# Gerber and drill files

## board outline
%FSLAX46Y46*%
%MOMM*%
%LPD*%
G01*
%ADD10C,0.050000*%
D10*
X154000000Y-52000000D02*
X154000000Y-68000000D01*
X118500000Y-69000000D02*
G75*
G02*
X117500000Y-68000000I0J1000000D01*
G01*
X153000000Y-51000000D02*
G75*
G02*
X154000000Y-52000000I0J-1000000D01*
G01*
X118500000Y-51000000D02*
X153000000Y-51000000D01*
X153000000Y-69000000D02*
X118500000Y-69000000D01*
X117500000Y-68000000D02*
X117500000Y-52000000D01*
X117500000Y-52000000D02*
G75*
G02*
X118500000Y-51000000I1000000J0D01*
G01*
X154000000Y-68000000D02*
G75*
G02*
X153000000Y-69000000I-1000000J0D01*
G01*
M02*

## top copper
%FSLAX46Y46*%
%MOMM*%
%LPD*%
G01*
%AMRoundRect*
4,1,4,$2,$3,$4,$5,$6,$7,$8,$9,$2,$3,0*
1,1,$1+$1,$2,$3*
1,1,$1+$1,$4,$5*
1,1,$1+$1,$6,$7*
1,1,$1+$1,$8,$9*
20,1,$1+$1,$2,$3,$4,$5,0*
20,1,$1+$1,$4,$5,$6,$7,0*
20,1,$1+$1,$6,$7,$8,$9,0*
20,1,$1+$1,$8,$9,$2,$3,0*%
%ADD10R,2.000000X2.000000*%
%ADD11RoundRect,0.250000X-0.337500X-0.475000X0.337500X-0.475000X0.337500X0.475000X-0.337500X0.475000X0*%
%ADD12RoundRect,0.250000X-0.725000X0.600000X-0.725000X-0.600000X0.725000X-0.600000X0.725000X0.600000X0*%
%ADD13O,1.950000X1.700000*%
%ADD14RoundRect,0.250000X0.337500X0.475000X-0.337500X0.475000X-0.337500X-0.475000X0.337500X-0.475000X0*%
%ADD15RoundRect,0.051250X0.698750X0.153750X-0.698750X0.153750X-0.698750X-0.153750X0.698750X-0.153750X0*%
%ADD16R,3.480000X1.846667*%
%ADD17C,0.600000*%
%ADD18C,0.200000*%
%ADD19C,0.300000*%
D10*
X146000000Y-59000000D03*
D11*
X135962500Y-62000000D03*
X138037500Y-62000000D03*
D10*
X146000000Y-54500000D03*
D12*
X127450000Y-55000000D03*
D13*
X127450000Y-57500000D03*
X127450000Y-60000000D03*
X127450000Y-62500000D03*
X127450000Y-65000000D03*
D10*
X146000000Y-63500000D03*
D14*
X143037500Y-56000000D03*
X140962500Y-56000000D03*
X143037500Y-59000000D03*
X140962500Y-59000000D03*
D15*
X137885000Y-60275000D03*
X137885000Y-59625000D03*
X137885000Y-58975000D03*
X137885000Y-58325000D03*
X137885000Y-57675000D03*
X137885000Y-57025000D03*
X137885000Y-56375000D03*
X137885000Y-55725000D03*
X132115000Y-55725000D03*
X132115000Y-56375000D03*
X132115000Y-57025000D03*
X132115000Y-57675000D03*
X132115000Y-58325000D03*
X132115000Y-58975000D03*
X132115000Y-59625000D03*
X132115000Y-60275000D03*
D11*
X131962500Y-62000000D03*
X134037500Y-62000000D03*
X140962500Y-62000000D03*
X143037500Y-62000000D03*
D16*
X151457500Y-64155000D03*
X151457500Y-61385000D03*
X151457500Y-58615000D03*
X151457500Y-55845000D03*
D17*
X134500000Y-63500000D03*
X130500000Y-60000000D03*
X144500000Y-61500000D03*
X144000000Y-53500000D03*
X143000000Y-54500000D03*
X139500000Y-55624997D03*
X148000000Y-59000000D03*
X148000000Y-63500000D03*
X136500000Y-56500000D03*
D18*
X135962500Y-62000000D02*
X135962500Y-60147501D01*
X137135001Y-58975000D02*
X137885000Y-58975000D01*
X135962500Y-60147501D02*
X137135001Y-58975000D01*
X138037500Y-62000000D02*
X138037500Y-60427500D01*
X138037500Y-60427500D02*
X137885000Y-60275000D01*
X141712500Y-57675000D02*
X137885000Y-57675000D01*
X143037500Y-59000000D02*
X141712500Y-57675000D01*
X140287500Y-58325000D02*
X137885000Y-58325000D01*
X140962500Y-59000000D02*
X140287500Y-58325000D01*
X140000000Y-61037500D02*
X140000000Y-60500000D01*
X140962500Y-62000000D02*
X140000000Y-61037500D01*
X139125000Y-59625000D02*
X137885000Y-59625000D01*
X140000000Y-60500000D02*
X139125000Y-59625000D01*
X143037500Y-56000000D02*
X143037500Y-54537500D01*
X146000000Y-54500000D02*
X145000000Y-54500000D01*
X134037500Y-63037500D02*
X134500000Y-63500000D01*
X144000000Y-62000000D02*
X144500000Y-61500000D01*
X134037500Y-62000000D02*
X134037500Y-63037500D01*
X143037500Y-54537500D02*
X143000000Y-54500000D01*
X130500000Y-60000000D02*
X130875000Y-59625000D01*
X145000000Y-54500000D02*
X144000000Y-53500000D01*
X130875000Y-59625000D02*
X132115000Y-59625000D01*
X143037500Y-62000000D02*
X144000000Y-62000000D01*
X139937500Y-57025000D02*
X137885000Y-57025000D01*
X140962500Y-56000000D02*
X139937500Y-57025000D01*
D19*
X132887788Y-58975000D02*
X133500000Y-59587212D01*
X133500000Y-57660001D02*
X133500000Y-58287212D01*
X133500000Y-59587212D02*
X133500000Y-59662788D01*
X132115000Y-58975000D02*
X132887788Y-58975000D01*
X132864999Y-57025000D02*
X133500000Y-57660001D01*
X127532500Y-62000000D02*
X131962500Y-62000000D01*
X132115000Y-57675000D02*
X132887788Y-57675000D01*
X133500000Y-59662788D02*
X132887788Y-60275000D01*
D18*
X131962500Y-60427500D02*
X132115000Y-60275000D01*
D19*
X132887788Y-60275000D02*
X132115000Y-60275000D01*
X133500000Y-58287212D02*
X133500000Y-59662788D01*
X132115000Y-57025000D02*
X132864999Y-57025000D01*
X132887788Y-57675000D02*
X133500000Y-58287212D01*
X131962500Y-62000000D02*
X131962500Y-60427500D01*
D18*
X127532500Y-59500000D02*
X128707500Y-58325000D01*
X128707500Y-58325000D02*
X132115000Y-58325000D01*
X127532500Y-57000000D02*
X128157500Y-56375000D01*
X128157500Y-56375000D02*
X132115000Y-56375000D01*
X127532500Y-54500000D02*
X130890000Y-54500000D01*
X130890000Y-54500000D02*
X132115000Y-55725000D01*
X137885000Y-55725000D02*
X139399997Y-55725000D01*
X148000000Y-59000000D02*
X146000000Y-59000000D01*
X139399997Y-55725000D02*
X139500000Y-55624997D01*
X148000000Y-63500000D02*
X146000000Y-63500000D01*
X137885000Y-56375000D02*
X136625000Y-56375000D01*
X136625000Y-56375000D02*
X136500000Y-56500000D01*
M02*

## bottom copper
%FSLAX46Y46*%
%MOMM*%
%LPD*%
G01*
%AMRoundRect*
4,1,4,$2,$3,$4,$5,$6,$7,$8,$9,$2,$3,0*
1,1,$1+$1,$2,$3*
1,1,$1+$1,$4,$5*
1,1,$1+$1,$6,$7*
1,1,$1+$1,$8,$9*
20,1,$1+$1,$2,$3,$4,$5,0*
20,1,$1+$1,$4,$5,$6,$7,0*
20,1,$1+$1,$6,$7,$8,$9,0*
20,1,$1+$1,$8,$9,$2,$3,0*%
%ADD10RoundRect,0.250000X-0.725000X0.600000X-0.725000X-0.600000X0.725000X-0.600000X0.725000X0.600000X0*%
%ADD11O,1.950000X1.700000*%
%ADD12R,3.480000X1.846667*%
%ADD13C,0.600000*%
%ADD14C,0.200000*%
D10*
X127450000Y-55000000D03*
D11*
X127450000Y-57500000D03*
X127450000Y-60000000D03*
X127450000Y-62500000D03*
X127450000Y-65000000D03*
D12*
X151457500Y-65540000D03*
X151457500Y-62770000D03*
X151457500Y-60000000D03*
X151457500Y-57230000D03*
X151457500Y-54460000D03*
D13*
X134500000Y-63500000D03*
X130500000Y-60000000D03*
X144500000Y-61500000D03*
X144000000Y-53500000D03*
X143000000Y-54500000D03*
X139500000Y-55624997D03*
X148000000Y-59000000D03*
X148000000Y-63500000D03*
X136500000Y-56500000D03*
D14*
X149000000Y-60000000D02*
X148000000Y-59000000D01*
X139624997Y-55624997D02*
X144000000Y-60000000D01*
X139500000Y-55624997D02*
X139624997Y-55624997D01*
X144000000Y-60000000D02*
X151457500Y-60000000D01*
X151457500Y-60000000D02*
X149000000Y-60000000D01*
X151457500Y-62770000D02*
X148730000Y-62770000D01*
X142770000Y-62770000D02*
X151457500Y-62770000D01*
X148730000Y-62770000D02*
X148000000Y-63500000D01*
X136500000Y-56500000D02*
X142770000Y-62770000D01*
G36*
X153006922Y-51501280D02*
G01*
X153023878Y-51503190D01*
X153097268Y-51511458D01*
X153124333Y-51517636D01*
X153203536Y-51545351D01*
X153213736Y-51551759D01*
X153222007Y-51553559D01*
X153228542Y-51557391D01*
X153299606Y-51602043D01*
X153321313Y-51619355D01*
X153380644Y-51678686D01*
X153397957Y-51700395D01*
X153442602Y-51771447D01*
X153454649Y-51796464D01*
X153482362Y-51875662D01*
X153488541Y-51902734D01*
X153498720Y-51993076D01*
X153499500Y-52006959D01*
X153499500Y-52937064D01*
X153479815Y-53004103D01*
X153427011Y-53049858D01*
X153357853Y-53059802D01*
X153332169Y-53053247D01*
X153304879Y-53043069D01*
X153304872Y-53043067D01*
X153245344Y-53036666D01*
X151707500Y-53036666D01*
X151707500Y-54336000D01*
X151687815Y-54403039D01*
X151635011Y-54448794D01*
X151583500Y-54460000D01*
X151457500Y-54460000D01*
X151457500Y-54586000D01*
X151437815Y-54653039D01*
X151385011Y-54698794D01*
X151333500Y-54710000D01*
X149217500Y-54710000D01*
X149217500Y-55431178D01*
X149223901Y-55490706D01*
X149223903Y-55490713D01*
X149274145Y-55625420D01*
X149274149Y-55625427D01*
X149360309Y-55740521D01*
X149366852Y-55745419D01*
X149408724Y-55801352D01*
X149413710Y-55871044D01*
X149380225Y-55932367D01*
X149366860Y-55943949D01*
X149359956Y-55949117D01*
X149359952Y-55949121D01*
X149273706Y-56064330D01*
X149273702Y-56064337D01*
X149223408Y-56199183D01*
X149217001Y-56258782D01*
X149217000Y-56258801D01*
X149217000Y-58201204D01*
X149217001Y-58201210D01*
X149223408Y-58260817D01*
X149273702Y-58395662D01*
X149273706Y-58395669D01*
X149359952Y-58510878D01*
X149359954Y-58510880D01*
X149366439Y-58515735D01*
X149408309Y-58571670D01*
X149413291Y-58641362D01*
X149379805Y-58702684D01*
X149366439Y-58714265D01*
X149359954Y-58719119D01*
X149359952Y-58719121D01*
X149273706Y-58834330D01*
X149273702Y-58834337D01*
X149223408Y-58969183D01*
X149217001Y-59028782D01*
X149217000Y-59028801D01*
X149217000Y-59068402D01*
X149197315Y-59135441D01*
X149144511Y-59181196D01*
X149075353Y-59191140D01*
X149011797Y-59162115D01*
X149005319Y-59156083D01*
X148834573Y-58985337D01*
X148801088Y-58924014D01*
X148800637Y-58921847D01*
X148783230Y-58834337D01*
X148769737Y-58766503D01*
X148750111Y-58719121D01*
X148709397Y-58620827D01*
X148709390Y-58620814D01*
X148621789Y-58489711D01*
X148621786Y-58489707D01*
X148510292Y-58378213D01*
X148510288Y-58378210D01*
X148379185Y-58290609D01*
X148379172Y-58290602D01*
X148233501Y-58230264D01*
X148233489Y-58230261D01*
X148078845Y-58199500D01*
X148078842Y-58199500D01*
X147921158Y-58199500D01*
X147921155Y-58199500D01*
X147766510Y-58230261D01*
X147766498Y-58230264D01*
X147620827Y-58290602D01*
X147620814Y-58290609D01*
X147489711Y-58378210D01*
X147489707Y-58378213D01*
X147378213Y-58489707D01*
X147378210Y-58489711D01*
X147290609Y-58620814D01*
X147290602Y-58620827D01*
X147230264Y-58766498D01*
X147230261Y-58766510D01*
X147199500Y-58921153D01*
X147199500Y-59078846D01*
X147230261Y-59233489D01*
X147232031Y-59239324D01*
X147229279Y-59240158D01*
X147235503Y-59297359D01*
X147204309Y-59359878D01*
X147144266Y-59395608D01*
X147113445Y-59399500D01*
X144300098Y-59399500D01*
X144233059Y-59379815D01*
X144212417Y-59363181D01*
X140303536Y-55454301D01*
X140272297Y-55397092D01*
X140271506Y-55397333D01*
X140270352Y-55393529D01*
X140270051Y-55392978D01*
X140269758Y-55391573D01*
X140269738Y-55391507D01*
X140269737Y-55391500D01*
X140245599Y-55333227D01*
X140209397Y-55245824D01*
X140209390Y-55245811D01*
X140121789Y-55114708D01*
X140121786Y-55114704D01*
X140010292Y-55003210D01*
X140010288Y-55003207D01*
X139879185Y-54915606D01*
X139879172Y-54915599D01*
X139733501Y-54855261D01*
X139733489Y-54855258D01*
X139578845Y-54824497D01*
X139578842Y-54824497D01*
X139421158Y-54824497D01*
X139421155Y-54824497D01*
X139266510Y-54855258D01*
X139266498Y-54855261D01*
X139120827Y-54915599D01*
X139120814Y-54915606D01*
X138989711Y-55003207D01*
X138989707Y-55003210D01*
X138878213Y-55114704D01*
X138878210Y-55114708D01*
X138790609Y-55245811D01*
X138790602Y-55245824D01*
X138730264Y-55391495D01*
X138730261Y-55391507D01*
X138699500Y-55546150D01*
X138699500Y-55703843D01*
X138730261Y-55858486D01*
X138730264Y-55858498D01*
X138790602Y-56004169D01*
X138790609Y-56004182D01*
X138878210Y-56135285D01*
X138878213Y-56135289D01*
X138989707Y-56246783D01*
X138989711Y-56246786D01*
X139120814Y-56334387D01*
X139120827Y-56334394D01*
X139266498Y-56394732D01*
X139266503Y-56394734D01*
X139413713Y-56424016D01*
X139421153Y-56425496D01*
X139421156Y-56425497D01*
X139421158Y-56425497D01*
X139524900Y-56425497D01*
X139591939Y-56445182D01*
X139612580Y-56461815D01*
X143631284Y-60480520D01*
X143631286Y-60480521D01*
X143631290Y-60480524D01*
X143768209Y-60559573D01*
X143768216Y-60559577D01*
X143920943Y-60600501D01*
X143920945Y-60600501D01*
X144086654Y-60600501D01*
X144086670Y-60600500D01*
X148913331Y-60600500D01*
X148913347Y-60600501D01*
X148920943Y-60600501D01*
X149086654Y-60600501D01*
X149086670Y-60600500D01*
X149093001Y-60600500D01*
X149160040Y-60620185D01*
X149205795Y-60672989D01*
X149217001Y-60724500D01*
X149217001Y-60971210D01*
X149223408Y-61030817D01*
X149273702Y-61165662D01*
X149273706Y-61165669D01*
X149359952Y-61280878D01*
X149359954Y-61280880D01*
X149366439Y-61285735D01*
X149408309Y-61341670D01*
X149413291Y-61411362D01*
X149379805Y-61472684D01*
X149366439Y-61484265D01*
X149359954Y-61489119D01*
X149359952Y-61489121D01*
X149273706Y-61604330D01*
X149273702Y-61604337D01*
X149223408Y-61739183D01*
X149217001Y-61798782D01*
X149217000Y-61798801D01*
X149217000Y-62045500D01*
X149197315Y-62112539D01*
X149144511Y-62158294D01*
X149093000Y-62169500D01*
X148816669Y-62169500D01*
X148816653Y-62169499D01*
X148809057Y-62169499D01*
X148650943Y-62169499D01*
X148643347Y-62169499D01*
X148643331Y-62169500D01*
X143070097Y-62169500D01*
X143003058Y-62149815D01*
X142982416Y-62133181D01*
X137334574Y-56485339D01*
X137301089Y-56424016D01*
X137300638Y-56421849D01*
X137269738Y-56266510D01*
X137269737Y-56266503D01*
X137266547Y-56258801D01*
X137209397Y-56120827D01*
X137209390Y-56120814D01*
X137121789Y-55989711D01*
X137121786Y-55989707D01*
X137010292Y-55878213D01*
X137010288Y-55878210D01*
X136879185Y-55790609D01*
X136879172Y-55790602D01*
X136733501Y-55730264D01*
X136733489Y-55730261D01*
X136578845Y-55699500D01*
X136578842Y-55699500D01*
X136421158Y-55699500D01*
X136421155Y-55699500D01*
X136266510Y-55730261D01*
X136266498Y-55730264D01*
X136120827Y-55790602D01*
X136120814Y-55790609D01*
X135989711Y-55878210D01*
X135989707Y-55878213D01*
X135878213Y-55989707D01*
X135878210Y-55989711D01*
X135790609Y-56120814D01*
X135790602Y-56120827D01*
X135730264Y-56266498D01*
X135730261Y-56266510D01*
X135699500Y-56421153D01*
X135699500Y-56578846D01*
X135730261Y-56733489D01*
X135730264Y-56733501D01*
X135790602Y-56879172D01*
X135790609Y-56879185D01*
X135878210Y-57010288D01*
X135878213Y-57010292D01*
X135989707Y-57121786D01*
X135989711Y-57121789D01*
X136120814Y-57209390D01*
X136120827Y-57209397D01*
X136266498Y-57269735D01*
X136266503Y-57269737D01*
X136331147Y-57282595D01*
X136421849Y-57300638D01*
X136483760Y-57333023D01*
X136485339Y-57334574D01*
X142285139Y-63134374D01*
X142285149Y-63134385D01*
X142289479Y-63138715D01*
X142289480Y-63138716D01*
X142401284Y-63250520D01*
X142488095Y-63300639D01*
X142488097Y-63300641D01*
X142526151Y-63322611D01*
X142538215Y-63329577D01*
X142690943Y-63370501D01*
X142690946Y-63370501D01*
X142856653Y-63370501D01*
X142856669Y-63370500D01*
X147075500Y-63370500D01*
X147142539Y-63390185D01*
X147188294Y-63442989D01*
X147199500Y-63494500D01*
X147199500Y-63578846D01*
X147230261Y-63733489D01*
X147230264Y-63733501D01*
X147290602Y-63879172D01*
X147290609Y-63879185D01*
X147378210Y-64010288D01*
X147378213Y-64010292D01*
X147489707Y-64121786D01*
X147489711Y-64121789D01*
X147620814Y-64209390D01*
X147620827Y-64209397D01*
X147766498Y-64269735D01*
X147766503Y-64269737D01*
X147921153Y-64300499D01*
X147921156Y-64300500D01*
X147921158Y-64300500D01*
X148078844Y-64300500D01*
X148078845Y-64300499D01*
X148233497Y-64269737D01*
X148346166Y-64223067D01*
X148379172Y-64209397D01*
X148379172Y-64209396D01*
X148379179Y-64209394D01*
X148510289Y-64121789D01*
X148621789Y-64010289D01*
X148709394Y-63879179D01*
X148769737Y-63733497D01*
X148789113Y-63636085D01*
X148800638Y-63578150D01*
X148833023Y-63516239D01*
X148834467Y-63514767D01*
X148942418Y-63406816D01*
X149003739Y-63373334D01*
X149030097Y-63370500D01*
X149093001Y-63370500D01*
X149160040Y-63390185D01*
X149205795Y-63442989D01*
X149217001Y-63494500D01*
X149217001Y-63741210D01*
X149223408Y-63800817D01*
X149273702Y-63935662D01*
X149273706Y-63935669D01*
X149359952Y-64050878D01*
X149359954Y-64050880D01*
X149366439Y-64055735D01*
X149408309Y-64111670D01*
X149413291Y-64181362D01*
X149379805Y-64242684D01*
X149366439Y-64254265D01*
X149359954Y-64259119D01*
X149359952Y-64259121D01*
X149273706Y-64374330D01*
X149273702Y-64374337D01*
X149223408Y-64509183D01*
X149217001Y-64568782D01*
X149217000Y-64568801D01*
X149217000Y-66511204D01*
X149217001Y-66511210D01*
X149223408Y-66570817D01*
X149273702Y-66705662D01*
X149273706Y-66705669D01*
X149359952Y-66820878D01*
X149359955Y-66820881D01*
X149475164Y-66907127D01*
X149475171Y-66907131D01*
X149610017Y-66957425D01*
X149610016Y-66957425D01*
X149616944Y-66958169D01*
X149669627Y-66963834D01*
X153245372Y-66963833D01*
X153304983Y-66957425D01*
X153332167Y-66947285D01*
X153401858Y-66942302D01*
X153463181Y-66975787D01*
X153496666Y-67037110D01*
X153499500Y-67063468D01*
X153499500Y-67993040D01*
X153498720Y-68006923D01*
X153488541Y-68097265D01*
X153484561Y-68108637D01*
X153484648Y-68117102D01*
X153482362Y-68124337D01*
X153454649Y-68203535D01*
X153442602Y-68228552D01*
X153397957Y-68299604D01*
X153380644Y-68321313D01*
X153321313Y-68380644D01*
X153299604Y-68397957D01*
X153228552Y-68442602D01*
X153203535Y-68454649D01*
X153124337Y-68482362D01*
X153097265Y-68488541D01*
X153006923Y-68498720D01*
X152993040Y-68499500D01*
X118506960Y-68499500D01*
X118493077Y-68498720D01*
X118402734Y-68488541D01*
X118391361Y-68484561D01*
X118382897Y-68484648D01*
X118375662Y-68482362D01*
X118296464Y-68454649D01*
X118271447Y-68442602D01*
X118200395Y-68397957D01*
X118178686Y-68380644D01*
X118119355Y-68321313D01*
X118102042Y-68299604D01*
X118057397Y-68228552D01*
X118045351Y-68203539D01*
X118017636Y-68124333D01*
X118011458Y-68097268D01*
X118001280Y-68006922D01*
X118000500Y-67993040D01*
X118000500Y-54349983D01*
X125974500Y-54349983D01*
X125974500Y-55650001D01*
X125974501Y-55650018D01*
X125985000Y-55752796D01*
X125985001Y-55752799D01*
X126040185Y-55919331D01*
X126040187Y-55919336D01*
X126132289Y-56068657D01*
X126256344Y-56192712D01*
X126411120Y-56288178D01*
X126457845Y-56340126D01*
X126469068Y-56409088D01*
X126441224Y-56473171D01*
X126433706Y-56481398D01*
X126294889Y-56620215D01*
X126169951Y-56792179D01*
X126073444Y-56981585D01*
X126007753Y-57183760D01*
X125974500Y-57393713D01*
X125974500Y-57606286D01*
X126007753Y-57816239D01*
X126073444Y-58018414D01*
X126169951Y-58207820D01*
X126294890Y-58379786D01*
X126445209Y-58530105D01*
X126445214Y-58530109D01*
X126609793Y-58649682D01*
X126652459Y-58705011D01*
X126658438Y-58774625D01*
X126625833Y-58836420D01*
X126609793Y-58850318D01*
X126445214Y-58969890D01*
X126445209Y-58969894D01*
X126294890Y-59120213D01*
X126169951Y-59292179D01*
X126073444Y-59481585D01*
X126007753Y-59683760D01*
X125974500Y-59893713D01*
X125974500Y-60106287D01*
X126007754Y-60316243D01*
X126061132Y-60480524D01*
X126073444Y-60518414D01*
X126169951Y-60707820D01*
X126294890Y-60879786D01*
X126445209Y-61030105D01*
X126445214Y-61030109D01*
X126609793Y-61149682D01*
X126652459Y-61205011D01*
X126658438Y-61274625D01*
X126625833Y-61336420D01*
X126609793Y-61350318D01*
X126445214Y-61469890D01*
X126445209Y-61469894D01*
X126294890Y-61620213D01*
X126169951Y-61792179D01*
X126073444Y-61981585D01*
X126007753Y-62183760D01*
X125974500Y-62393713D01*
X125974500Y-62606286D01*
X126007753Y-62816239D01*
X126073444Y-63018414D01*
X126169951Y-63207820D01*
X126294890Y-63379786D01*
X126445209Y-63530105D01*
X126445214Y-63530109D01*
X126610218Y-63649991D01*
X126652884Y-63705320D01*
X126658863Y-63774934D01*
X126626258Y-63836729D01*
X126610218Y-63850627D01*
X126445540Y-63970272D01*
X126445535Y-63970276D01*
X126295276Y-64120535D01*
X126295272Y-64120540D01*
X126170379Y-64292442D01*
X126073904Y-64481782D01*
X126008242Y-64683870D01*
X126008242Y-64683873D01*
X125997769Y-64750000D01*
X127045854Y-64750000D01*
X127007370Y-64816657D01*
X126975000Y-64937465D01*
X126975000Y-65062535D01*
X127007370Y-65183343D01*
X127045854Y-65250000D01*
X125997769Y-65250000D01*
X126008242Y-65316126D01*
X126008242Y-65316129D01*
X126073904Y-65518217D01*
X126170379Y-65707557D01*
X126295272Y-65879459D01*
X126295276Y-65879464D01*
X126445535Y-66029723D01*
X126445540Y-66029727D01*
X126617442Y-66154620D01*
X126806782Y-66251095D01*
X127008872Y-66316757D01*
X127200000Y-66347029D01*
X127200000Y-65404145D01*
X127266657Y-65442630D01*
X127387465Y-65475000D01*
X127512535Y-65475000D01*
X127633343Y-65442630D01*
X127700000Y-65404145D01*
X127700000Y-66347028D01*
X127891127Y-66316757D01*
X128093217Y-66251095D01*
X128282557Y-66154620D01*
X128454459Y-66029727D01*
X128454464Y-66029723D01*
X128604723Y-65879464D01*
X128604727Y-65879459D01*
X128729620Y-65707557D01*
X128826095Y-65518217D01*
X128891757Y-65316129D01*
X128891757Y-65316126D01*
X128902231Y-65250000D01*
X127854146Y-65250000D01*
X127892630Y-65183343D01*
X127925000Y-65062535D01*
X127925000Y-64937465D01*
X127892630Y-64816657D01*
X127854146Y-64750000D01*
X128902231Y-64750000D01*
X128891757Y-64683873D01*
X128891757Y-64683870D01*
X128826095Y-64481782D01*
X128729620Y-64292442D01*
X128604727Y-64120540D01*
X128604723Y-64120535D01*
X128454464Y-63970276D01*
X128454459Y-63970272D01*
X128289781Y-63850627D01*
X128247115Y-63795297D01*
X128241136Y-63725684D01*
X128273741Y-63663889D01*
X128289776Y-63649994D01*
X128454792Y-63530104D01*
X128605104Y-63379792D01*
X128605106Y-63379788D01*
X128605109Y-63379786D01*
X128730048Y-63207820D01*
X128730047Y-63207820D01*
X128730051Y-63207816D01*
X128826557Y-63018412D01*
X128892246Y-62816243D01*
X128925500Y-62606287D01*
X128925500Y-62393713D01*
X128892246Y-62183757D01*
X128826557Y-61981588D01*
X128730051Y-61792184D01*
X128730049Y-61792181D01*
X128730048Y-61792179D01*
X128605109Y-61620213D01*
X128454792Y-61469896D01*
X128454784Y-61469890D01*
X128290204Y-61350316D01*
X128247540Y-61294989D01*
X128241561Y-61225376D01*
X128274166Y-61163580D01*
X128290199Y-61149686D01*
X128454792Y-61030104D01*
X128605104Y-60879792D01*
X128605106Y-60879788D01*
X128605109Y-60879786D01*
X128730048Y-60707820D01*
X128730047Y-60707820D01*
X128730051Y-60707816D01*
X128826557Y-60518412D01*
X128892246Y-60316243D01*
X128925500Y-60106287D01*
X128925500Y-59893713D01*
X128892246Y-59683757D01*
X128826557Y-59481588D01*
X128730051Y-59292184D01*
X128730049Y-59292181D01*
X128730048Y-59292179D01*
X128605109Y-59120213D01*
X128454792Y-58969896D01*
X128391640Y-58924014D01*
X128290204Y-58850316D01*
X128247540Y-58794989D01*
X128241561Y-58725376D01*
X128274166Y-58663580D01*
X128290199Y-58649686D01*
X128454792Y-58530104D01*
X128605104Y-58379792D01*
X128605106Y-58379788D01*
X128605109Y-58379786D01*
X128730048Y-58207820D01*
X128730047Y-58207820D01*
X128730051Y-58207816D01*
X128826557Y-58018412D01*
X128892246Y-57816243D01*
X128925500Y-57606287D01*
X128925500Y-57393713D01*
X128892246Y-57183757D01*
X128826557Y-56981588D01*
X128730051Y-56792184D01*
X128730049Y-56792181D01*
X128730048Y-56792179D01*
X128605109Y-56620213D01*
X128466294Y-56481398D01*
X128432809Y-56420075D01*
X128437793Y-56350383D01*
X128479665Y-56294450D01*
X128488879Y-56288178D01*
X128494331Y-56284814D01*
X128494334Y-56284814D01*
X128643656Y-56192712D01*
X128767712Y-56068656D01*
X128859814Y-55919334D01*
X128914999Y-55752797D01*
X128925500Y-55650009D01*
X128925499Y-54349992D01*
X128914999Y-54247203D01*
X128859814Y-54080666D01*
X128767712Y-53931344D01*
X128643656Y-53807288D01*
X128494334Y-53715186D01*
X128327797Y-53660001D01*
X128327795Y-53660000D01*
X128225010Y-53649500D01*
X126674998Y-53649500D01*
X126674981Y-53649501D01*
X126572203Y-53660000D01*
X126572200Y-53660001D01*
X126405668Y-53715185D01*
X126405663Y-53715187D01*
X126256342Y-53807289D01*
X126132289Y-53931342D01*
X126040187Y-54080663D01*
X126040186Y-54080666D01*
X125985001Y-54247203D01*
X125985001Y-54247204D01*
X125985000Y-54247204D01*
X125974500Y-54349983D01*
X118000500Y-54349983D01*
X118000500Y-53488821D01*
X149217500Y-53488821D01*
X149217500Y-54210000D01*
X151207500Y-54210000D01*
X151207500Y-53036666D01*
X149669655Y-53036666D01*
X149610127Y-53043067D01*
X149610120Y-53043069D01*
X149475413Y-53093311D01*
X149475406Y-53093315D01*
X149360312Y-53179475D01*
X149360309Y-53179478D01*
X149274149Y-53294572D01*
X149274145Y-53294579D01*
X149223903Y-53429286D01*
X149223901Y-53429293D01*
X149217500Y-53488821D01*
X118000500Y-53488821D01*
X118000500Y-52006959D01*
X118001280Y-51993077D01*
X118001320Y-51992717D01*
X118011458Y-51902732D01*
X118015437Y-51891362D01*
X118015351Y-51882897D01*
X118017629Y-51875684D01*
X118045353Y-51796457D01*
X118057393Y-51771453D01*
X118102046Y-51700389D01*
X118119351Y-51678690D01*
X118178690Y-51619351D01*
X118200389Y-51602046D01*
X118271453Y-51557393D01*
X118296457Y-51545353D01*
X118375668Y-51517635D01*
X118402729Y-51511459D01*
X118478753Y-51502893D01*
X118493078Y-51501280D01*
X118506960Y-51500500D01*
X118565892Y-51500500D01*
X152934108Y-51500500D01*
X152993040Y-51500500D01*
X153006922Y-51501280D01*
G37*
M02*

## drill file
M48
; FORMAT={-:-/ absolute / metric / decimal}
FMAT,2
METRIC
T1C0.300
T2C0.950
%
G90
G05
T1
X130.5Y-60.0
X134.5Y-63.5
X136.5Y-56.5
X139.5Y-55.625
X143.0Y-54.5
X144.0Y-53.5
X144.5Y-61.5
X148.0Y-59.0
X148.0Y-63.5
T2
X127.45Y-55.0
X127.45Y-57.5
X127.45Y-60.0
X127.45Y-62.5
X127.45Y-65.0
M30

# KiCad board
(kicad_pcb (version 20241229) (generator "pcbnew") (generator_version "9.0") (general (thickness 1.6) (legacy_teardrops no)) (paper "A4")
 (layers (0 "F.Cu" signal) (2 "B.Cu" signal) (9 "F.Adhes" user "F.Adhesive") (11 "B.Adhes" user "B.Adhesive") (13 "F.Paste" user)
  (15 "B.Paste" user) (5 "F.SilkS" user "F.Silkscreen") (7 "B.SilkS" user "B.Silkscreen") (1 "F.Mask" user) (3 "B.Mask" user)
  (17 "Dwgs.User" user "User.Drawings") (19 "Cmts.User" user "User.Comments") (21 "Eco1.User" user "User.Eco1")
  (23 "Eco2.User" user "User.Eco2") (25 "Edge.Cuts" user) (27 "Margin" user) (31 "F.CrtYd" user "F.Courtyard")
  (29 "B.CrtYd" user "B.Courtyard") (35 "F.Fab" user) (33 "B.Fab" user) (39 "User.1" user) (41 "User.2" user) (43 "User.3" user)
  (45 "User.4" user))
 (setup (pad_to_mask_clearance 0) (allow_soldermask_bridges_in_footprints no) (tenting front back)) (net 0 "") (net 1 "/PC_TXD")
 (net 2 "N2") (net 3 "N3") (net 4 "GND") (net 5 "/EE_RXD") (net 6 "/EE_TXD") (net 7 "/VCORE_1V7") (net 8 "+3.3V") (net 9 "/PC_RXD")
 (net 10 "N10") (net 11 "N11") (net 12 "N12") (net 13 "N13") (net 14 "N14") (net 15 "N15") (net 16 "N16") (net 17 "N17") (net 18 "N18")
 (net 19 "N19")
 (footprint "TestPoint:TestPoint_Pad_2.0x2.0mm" (layer "F.Cu") (at 146 59)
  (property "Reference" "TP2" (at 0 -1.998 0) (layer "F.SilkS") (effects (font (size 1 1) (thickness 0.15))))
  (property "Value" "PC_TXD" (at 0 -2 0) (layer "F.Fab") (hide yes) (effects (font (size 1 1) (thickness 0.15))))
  (pad "1" smd rect (at 0 0) (size 2 2) (layers "F.Cu" "F.Mask") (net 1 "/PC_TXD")))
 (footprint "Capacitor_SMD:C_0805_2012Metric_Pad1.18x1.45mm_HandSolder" (layer "F.Cu") (at 137 62)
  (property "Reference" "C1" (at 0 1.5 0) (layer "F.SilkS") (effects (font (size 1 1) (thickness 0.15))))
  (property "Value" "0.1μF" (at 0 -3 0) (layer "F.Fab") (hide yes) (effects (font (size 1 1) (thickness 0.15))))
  (pad "1" smd roundrect (at -1.0375 0) (size 1.175 1.45) (layers "F.Cu" "F.Mask" "F.Paste") (roundrect_rratio 0.212766) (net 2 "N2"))
  (pad "2" smd roundrect (at 1.0375 0) (size 1.175 1.45) (layers "F.Cu" "F.Mask" "F.Paste") (roundrect_rratio 0.212766) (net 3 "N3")))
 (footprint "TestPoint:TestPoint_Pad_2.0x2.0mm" (layer "F.Cu") (at 146 54.5)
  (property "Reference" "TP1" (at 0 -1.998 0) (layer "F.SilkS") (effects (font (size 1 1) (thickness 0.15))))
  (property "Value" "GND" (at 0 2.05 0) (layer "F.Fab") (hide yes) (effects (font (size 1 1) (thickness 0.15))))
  (pad "1" smd rect (at 0 0) (size 2 2) (layers "F.Cu" "F.Mask") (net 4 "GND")))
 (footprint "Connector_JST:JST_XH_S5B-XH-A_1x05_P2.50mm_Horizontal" (layer "F.Cu") (at 127.45 55 -90)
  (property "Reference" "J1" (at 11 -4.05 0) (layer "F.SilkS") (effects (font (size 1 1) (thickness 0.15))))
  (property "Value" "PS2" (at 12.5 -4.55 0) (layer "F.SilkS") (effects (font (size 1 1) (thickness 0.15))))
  (pad "1" thru_hole roundrect (at 0 0 270) (size 1.7 1.95) (drill 0.95) (layers "*.Cu" "*.Mask") (remove_unused_layers no)
   (roundrect_rratio 0.147059) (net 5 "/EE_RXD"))
  (pad "2" thru_hole oval (at 2.5 0 270) (size 1.7 1.95) (drill 0.95) (layers "*.Cu" "*.Mask") (remove_unused_layers no) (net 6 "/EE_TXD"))
  (pad "3" thru_hole oval (at 5 0 270) (size 1.7 1.95) (drill 0.95) (layers "*.Cu" "*.Mask") (remove_unused_layers no) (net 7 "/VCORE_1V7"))
  (pad "4" thru_hole oval (at 7.5 0 270) (size 1.7 1.95) (drill 0.95) (layers "*.Cu" "*.Mask") (remove_unused_layers no) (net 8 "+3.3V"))
  (pad "5" thru_hole oval (at 10 0 270) (size 1.7 1.95) (drill 0.95) (layers "*.Cu" "*.Mask") (remove_unused_layers no) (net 4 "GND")))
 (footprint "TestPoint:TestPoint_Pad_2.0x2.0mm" (layer "F.Cu") (at 146 63.5)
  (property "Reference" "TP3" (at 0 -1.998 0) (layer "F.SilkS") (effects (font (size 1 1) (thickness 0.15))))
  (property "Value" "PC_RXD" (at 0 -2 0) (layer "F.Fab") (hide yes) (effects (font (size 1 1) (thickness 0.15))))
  (pad "1" smd rect (at 0 0) (size 2 2) (layers "F.Cu" "F.Mask") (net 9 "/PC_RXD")))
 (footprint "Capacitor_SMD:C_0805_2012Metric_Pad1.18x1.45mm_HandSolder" (layer "F.Cu") (at 142 56 180)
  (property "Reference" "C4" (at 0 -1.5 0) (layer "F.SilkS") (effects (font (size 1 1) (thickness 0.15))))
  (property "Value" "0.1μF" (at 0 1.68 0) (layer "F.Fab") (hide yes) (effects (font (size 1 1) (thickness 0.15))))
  (pad "1" smd roundrect (at -1.0375 0 180) (size 1.175 1.45) (layers "F.Cu" "F.Mask" "F.Paste") (roundrect_rratio 0.212766) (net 4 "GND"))
  (pad "2" smd roundrect (at 1.0375 0 180) (size 1.175 1.45) (layers "F.Cu" "F.Mask" "F.Paste") (roundrect_rratio 0.212766) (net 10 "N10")))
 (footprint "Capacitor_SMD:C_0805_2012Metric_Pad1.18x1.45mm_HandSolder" (layer "F.Cu") (at 142 59 180)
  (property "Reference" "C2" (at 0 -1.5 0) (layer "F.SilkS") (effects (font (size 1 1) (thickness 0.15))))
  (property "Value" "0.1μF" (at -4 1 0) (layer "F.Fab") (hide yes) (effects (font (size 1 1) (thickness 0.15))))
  (pad "1" smd roundrect (at -1.0375 0 180) (size 1.175 1.45) (layers "F.Cu" "F.Mask" "F.Paste") (roundrect_rratio 0.212766) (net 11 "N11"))
  (pad "2" smd roundrect (at 1.0375 0 180) (size 1.175 1.45) (layers "F.Cu" "F.Mask" "F.Paste") (roundrect_rratio 0.212766) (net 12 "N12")))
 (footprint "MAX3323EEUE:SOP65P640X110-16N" (layer "F.Cu") (at 135 58 180)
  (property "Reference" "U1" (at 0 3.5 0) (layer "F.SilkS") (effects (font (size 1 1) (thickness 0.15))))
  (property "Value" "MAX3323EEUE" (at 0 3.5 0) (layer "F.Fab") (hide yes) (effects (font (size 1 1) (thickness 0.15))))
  (pad "1" smd roundrect (at -2.885 -2.275 180) (size 1.5 0.41) (layers "F.Cu" "F.Mask" "F.Paste") (roundrect_rratio 0.125) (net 3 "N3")
   (solder_mask_margin 0.102))
  (pad "2" smd roundrect (at -2.885 -1.625 180) (size 1.5 0.41) (layers "F.Cu" "F.Mask" "F.Paste") (roundrect_rratio 0.125) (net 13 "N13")
   (solder_mask_margin 0.102))
  (pad "3" smd roundrect (at -2.885 -0.975 180) (size 1.5 0.41) (layers "F.Cu" "F.Mask" "F.Paste") (roundrect_rratio 0.125) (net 2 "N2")
   (solder_mask_margin 0.102))
  (pad "4" smd roundrect (at -2.885 -0.325 180) (size 1.5 0.41) (layers "F.Cu" "F.Mask" "F.Paste") (roundrect_rratio 0.125) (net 12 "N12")
   (solder_mask_margin 0.102))
  (pad "5" smd roundrect (at -2.885 0.325 180) (size 1.5 0.41) (layers "F.Cu" "F.Mask" "F.Paste") (roundrect_rratio 0.125) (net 11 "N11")
   (solder_mask_margin 0.102))
  (pad "6" smd roundrect (at -2.885 0.975 180) (size 1.5 0.41) (layers "F.Cu" "F.Mask" "F.Paste") (roundrect_rratio 0.125) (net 10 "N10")
   (solder_mask_margin 0.102))
  (pad "7" smd roundrect (at -2.885 1.625 180) (size 1.5 0.41) (layers "F.Cu" "F.Mask" "F.Paste") (roundrect_rratio 0.125) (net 9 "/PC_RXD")
   (solder_mask_margin 0.102))
  (pad "8" smd roundrect (at -2.885 2.275 180) (size 1.5 0.41) (layers "F.Cu" "F.Mask" "F.Paste") (roundrect_rratio 0.125) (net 1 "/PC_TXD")
   (solder_mask_margin 0.102))
  (pad "9" smd roundrect (at 2.885 2.275 180) (size 1.5 0.41) (layers "F.Cu" "F.Mask" "F.Paste") (roundrect_rratio 0.125) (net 5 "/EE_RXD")
   (solder_mask_margin 0.102))
  (pad "10" smd roundrect (at 2.885 1.625 180) (size 1.5 0.41) (layers "F.Cu" "F.Mask" "F.Paste") (roundrect_rratio 0.125) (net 6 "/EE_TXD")
   (solder_mask_margin 0.102))
  (pad "11" smd roundrect (at 2.885 0.975 180) (size 1.5 0.41) (layers "F.Cu" "F.Mask" "F.Paste") (roundrect_rratio 0.125) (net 8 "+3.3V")
   (solder_mask_margin 0.102))
  (pad "12" smd roundrect (at 2.885 0.325 180) (size 1.5 0.41) (layers "F.Cu" "F.Mask" "F.Paste") (roundrect_rratio 0.125) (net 8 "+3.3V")
   (solder_mask_margin 0.102))
  (pad "13" smd roundrect (at 2.885 -0.325 180) (size 1.5 0.41) (layers "F.Cu" "F.Mask" "F.Paste") (roundrect_rratio 0.125)
   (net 7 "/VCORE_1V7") (solder_mask_margin 0.102))
  (pad "14" smd roundrect (at 2.885 -0.975 180) (size 1.5 0.41) (layers "F.Cu" "F.Mask" "F.Paste") (roundrect_rratio 0.125) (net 8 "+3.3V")
   (solder_mask_margin 0.102))
  (pad "15" smd roundrect (at 2.885 -1.625 180) (size 1.5 0.41) (layers "F.Cu" "F.Mask" "F.Paste") (roundrect_rratio 0.125) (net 4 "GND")
   (solder_mask_margin 0.102))
  (pad "16" smd roundrect (at 2.885 -2.275 180) (size 1.5 0.41) (layers "F.Cu" "F.Mask" "F.Paste") (roundrect_rratio 0.125) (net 8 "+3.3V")
   (solder_mask_margin 0.102)))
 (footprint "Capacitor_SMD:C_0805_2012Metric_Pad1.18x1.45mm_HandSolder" (layer "F.Cu") (at 133 62)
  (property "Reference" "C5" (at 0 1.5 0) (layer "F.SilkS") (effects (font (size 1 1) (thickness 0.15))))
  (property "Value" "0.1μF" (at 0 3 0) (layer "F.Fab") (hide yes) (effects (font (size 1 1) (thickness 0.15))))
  (pad "1" smd roundrect (at -1.0375 0) (size 1.175 1.45) (layers "F.Cu" "F.Mask" "F.Paste") (roundrect_rratio 0.212766) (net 8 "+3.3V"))
  (pad "2" smd roundrect (at 1.0375 0) (size 1.175 1.45) (layers "F.Cu" "F.Mask" "F.Paste") (roundrect_rratio 0.212766) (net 4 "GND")))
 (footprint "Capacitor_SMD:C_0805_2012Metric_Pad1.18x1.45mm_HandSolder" (layer "F.Cu") (at 142 62)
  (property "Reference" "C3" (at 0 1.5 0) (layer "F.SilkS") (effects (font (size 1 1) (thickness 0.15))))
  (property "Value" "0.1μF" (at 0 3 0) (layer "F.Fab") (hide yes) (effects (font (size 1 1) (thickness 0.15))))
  (pad "1" smd roundrect (at -1.0375 0) (size 1.175 1.45) (layers "F.Cu" "F.Mask" "F.Paste") (roundrect_rratio 0.212766) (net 13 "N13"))
  (pad "2" smd roundrect (at 1.0375 0) (size 1.175 1.45) (layers "F.Cu" "F.Mask" "F.Paste") (roundrect_rratio 0.212766) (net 4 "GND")))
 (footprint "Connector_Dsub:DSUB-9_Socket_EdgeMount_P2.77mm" (layer "B.Cu") (at 151.4575 60 -90)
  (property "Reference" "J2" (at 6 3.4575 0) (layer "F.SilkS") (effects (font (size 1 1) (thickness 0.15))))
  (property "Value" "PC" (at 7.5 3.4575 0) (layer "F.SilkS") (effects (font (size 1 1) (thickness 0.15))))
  (pad "1" smd rect (at 5.54 0 270) (size 1.846667 3.48) (layers "B.Cu" "B.Mask" "B.Paste") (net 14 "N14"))
  (pad "2" smd rect (at 2.77 0 270) (size 1.846667 3.48) (layers "B.Cu" "B.Mask" "B.Paste") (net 9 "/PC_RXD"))
  (pad "3" smd rect (at 0 0 270) (size 1.846667 3.48) (layers "B.Cu" "B.Mask" "B.Paste") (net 1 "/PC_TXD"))
  (pad "4" smd rect (at -2.77 0 270) (size 1.846667 3.48) (layers "B.Cu" "B.Mask" "B.Paste") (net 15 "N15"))
  (pad "5" smd rect (at -5.54 0 270) (size 1.846667 3.48) (layers "B.Cu" "B.Mask" "B.Paste") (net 4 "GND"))
  (pad "6" smd rect (at 4.155 0 270) (size 1.846667 3.48) (layers "F.Cu" "F.Mask" "F.Paste") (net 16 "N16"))
  (pad "7" smd rect (at 1.385 0 270) (size 1.846667 3.48) (layers "F.Cu" "F.Mask" "F.Paste") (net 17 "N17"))
  (pad "8" smd rect (at -1.385 0 270) (size 1.846667 3.48) (layers "F.Cu" "F.Mask" "F.Paste") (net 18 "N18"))
  (pad "9" smd rect (at -4.155 0 270) (size 1.846667 3.48) (layers "F.Cu" "F.Mask" "F.Paste") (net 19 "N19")))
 (gr_line (start 154 52) (end 154 68) (stroke (width 0.05) (type default)) (layer "Edge.Cuts"))
 (gr_arc (start 118.5 69) (mid 117.792893 68.707107) (end 117.5 68) (stroke (width 0.05) (type default)) (layer "Edge.Cuts"))
 (gr_arc (start 153 51) (mid 153.707107 51.292893) (end 154 52) (stroke (width 0.05) (type default)) (layer "Edge.Cuts"))
 (gr_line (start 118.5 51) (end 153 51) (stroke (width 0.05) (type default)) (layer "Edge.Cuts"))
 (gr_line (start 153 69) (end 118.5 69) (stroke (width 0.05) (type default)) (layer "Edge.Cuts"))
 (gr_line (start 117.5 68) (end 117.5 52) (stroke (width 0.05) (type default)) (layer "Edge.Cuts"))
 (gr_arc (start 117.5 52) (mid 117.792893 51.292893) (end 118.5 51) (stroke (width 0.05) (type default)) (layer "Edge.Cuts"))
 (gr_arc (start 154 68) (mid 153.707107 68.707107) (end 153 69) (stroke (width 0.05) (type default)) (layer "Edge.Cuts"))
 (segment (start 135.9625 62) (end 135.9625 60.147501) (width 0.2) (layer "F.Cu") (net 2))
 (segment (start 137.135001 58.975) (end 137.885 58.975) (width 0.2) (layer "F.Cu") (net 2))
 (segment (start 135.9625 60.147501) (end 137.135001 58.975) (width 0.2) (layer "F.Cu") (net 2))
 (segment (start 138.0375 62) (end 138.0375 60.4275) (width 0.2) (layer "F.Cu") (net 3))
 (segment (start 138.0375 60.4275) (end 137.885 60.275) (width 0.2) (layer "F.Cu") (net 3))
 (segment (start 141.7125 57.675) (end 137.885 57.675) (width 0.2) (layer "F.Cu") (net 11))
 (segment (start 143.0375 59) (end 141.7125 57.675) (width 0.2) (layer "F.Cu") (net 11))
 (segment (start 140.2875 58.325) (end 137.885 58.325) (width 0.2) (layer "F.Cu") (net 12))
 (segment (start 140.9625 59) (end 140.2875 58.325) (width 0.2) (layer "F.Cu") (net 12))
 (segment (start 140 61.0375) (end 140 60.5) (width 0.2) (layer "F.Cu") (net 13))
 (segment (start 140.9625 62) (end 140 61.0375) (width 0.2) (layer "F.Cu") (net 13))
 (segment (start 139.125 59.625) (end 137.885 59.625) (width 0.2) (layer "F.Cu") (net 13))
 (segment (start 140 60.5) (end 139.125 59.625) (width 0.2) (layer "F.Cu") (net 13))
 (segment (start 143.0375 56) (end 143.0375 54.5375) (width 0.2) (layer "F.Cu") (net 4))
 (segment (start 146 54.5) (end 145 54.5) (width 0.2) (layer "F.Cu") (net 4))
 (segment (start 134.0375 63.0375) (end 134.5 63.5) (width 0.2) (layer "F.Cu") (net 4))
 (segment (start 144 62) (end 144.5 61.5) (width 0.2) (layer "F.Cu") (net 4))
 (segment (start 134.0375 62) (end 134.0375 63.0375) (width 0.2) (layer "F.Cu") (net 4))
 (segment (start 143.0375 54.5375) (end 143 54.5) (width 0.2) (layer "F.Cu") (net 4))
 (segment (start 130.5 60) (end 130.875 59.625) (width 0.2) (layer "F.Cu") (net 4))
 (segment (start 145 54.5) (end 144 53.5) (width 0.2) (layer "F.Cu") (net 4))
 (segment (start 130.875 59.625) (end 132.115 59.625) (width 0.2) (layer "F.Cu") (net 4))
 (segment (start 143.0375 62) (end 144 62) (width 0.2) (layer "F.Cu") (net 4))
 (via (at 134.5 63.5) (size 0.6) (drill 0.3) (layers "F.Cu" "B.Cu") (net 4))
 (via (at 130.5 60) (size 0.6) (drill 0.3) (layers "F.Cu" "B.Cu") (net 4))
 (via (at 144.5 61.5) (size 0.6) (drill 0.3) (layers "F.Cu" "B.Cu") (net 4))
 (via (at 144 53.5) (size 0.6) (drill 0.3) (layers "F.Cu" "B.Cu") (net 4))
 (via (at 143 54.5) (size 0.6) (drill 0.3) (layers "F.Cu" "B.Cu") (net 4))
 (segment (start 139.9375 57.025) (end 137.885 57.025) (width 0.2) (layer "F.Cu") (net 10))
 (segment (start 140.9625 56) (end 139.9375 57.025) (width 0.2) (layer "F.Cu") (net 10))
 (segment (start 132.887788 58.975) (end 133.5 59.587212) (width 0.3) (layer "F.Cu") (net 8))
 (segment (start 133.5 57.660001) (end 133.5 58.287212) (width 0.3) (layer "F.Cu") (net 8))
 (segment (start 133.5 59.587212) (end 133.5 59.662788) (width 0.3) (layer "F.Cu") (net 8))
 (segment (start 132.115 58.975) (end 132.887788 58.975) (width 0.3) (layer "F.Cu") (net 8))
 (segment (start 132.864999 57.025) (end 133.5 57.660001) (width 0.3) (layer "F.Cu") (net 8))
 (segment (start 127.5325 62) (end 131.9625 62) (width 0.3) (layer "F.Cu") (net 8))
 (segment (start 132.115 57.675) (end 132.887788 57.675) (width 0.3) (layer "F.Cu") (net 8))
 (segment (start 133.5 59.662788) (end 132.887788 60.275) (width 0.3) (layer "F.Cu") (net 8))
 (segment (start 131.9625 60.4275) (end 132.115 60.275) (width 0.2) (layer "F.Cu") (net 8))
 (segment (start 132.887788 60.275) (end 132.115 60.275) (width 0.3) (layer "F.Cu") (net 8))
 (segment (start 133.5 58.287212) (end 133.5 59.662788) (width 0.3) (layer "F.Cu") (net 8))
 (segment (start 132.115 57.025) (end 132.864999 57.025) (width 0.3) (layer "F.Cu") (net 8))
 (segment (start 132.887788 57.675) (end 133.5 58.287212) (width 0.3) (layer "F.Cu") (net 8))
 (segment (start 131.9625 62) (end 131.9625 60.4275) (width 0.3) (layer "F.Cu") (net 8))
 (segment (start 127.5325 59.5) (end 128.7075 58.325) (width 0.2) (layer "F.Cu") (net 7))
 (segment (start 128.7075 58.325) (end 132.115 58.325) (width 0.2) (layer "F.Cu") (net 7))
 (segment (start 127.5325 57) (end 128.1575 56.375) (width 0.2) (layer "F.Cu") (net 6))
 (segment (start 128.1575 56.375) (end 132.115 56.375) (width 0.2) (layer "F.Cu") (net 6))
 (segment (start 127.5325 54.5) (end 130.89 54.5) (width 0.2) (layer "F.Cu") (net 5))
 (segment (start 130.89 54.5) (end 132.115 55.725) (width 0.2) (layer "F.Cu") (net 5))
 (segment (start 137.885 55.725) (end 139.399997 55.725) (width 0.2) (layer "F.Cu") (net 1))
 (segment (start 148 59) (end 146 59) (width 0.2) (layer "F.Cu") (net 1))
 (segment (start 139.399997 55.725) (end 139.5 55.624997) (width 0.2) (layer "F.Cu") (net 1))
 (via (at 139.5 55.624997) (size 0.6) (drill 0.3) (layers "F.Cu" "B.Cu") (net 1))
 (via (at 148 59) (size 0.6) (drill 0.3) (layers "F.Cu" "B.Cu") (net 1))
 (segment (start 149 60) (end 148 59) (width 0.2) (layer "B.Cu") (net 1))
 (segment (start 139.624997 55.624997) (end 144 60) (width 0.2) (layer "B.Cu") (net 1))
 (segment (start 139.5 55.624997) (end 139.624997 55.624997) (width 0.2) (layer "B.Cu") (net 1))
 (segment (start 144 60) (end 151.4575 60) (width 0.2) (layer "B.Cu") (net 1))
 (segment (start 151.4575 60) (end 149 60) (width 0.2) (layer "B.Cu") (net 1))
 (segment (start 148 63.5) (end 146 63.5) (width 0.2) (layer "F.Cu") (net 9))
 (segment (start 137.885 56.375) (end 136.625 56.375) (width 0.2) (layer "F.Cu") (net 9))
 (segment (start 136.625 56.375) (end 136.5 56.5) (width 0.2) (layer "F.Cu") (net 9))
 (via (at 148 63.5) (size 0.6) (drill 0.3) (layers "F.Cu" "B.Cu") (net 9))
 (via (at 136.5 56.5) (size 0.6) (drill 0.3) (layers "F.Cu" "B.Cu") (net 9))
 (segment (start 151.4575 62.77) (end 148.73 62.77) (width 0.2) (layer "B.Cu") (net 9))
 (segment (start 142.77 62.77) (end 151.4575 62.77) (width 0.2) (layer "B.Cu") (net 9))
 (segment (start 148.73 62.77) (end 148 63.5) (width 0.2) (layer "B.Cu") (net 9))
 (segment (start 136.5 56.5) (end 142.77 62.77) (width 0.2) (layer "B.Cu") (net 9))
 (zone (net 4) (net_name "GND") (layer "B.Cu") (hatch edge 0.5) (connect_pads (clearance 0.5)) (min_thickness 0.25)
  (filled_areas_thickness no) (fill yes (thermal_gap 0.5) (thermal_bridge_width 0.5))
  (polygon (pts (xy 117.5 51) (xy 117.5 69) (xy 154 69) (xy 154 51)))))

